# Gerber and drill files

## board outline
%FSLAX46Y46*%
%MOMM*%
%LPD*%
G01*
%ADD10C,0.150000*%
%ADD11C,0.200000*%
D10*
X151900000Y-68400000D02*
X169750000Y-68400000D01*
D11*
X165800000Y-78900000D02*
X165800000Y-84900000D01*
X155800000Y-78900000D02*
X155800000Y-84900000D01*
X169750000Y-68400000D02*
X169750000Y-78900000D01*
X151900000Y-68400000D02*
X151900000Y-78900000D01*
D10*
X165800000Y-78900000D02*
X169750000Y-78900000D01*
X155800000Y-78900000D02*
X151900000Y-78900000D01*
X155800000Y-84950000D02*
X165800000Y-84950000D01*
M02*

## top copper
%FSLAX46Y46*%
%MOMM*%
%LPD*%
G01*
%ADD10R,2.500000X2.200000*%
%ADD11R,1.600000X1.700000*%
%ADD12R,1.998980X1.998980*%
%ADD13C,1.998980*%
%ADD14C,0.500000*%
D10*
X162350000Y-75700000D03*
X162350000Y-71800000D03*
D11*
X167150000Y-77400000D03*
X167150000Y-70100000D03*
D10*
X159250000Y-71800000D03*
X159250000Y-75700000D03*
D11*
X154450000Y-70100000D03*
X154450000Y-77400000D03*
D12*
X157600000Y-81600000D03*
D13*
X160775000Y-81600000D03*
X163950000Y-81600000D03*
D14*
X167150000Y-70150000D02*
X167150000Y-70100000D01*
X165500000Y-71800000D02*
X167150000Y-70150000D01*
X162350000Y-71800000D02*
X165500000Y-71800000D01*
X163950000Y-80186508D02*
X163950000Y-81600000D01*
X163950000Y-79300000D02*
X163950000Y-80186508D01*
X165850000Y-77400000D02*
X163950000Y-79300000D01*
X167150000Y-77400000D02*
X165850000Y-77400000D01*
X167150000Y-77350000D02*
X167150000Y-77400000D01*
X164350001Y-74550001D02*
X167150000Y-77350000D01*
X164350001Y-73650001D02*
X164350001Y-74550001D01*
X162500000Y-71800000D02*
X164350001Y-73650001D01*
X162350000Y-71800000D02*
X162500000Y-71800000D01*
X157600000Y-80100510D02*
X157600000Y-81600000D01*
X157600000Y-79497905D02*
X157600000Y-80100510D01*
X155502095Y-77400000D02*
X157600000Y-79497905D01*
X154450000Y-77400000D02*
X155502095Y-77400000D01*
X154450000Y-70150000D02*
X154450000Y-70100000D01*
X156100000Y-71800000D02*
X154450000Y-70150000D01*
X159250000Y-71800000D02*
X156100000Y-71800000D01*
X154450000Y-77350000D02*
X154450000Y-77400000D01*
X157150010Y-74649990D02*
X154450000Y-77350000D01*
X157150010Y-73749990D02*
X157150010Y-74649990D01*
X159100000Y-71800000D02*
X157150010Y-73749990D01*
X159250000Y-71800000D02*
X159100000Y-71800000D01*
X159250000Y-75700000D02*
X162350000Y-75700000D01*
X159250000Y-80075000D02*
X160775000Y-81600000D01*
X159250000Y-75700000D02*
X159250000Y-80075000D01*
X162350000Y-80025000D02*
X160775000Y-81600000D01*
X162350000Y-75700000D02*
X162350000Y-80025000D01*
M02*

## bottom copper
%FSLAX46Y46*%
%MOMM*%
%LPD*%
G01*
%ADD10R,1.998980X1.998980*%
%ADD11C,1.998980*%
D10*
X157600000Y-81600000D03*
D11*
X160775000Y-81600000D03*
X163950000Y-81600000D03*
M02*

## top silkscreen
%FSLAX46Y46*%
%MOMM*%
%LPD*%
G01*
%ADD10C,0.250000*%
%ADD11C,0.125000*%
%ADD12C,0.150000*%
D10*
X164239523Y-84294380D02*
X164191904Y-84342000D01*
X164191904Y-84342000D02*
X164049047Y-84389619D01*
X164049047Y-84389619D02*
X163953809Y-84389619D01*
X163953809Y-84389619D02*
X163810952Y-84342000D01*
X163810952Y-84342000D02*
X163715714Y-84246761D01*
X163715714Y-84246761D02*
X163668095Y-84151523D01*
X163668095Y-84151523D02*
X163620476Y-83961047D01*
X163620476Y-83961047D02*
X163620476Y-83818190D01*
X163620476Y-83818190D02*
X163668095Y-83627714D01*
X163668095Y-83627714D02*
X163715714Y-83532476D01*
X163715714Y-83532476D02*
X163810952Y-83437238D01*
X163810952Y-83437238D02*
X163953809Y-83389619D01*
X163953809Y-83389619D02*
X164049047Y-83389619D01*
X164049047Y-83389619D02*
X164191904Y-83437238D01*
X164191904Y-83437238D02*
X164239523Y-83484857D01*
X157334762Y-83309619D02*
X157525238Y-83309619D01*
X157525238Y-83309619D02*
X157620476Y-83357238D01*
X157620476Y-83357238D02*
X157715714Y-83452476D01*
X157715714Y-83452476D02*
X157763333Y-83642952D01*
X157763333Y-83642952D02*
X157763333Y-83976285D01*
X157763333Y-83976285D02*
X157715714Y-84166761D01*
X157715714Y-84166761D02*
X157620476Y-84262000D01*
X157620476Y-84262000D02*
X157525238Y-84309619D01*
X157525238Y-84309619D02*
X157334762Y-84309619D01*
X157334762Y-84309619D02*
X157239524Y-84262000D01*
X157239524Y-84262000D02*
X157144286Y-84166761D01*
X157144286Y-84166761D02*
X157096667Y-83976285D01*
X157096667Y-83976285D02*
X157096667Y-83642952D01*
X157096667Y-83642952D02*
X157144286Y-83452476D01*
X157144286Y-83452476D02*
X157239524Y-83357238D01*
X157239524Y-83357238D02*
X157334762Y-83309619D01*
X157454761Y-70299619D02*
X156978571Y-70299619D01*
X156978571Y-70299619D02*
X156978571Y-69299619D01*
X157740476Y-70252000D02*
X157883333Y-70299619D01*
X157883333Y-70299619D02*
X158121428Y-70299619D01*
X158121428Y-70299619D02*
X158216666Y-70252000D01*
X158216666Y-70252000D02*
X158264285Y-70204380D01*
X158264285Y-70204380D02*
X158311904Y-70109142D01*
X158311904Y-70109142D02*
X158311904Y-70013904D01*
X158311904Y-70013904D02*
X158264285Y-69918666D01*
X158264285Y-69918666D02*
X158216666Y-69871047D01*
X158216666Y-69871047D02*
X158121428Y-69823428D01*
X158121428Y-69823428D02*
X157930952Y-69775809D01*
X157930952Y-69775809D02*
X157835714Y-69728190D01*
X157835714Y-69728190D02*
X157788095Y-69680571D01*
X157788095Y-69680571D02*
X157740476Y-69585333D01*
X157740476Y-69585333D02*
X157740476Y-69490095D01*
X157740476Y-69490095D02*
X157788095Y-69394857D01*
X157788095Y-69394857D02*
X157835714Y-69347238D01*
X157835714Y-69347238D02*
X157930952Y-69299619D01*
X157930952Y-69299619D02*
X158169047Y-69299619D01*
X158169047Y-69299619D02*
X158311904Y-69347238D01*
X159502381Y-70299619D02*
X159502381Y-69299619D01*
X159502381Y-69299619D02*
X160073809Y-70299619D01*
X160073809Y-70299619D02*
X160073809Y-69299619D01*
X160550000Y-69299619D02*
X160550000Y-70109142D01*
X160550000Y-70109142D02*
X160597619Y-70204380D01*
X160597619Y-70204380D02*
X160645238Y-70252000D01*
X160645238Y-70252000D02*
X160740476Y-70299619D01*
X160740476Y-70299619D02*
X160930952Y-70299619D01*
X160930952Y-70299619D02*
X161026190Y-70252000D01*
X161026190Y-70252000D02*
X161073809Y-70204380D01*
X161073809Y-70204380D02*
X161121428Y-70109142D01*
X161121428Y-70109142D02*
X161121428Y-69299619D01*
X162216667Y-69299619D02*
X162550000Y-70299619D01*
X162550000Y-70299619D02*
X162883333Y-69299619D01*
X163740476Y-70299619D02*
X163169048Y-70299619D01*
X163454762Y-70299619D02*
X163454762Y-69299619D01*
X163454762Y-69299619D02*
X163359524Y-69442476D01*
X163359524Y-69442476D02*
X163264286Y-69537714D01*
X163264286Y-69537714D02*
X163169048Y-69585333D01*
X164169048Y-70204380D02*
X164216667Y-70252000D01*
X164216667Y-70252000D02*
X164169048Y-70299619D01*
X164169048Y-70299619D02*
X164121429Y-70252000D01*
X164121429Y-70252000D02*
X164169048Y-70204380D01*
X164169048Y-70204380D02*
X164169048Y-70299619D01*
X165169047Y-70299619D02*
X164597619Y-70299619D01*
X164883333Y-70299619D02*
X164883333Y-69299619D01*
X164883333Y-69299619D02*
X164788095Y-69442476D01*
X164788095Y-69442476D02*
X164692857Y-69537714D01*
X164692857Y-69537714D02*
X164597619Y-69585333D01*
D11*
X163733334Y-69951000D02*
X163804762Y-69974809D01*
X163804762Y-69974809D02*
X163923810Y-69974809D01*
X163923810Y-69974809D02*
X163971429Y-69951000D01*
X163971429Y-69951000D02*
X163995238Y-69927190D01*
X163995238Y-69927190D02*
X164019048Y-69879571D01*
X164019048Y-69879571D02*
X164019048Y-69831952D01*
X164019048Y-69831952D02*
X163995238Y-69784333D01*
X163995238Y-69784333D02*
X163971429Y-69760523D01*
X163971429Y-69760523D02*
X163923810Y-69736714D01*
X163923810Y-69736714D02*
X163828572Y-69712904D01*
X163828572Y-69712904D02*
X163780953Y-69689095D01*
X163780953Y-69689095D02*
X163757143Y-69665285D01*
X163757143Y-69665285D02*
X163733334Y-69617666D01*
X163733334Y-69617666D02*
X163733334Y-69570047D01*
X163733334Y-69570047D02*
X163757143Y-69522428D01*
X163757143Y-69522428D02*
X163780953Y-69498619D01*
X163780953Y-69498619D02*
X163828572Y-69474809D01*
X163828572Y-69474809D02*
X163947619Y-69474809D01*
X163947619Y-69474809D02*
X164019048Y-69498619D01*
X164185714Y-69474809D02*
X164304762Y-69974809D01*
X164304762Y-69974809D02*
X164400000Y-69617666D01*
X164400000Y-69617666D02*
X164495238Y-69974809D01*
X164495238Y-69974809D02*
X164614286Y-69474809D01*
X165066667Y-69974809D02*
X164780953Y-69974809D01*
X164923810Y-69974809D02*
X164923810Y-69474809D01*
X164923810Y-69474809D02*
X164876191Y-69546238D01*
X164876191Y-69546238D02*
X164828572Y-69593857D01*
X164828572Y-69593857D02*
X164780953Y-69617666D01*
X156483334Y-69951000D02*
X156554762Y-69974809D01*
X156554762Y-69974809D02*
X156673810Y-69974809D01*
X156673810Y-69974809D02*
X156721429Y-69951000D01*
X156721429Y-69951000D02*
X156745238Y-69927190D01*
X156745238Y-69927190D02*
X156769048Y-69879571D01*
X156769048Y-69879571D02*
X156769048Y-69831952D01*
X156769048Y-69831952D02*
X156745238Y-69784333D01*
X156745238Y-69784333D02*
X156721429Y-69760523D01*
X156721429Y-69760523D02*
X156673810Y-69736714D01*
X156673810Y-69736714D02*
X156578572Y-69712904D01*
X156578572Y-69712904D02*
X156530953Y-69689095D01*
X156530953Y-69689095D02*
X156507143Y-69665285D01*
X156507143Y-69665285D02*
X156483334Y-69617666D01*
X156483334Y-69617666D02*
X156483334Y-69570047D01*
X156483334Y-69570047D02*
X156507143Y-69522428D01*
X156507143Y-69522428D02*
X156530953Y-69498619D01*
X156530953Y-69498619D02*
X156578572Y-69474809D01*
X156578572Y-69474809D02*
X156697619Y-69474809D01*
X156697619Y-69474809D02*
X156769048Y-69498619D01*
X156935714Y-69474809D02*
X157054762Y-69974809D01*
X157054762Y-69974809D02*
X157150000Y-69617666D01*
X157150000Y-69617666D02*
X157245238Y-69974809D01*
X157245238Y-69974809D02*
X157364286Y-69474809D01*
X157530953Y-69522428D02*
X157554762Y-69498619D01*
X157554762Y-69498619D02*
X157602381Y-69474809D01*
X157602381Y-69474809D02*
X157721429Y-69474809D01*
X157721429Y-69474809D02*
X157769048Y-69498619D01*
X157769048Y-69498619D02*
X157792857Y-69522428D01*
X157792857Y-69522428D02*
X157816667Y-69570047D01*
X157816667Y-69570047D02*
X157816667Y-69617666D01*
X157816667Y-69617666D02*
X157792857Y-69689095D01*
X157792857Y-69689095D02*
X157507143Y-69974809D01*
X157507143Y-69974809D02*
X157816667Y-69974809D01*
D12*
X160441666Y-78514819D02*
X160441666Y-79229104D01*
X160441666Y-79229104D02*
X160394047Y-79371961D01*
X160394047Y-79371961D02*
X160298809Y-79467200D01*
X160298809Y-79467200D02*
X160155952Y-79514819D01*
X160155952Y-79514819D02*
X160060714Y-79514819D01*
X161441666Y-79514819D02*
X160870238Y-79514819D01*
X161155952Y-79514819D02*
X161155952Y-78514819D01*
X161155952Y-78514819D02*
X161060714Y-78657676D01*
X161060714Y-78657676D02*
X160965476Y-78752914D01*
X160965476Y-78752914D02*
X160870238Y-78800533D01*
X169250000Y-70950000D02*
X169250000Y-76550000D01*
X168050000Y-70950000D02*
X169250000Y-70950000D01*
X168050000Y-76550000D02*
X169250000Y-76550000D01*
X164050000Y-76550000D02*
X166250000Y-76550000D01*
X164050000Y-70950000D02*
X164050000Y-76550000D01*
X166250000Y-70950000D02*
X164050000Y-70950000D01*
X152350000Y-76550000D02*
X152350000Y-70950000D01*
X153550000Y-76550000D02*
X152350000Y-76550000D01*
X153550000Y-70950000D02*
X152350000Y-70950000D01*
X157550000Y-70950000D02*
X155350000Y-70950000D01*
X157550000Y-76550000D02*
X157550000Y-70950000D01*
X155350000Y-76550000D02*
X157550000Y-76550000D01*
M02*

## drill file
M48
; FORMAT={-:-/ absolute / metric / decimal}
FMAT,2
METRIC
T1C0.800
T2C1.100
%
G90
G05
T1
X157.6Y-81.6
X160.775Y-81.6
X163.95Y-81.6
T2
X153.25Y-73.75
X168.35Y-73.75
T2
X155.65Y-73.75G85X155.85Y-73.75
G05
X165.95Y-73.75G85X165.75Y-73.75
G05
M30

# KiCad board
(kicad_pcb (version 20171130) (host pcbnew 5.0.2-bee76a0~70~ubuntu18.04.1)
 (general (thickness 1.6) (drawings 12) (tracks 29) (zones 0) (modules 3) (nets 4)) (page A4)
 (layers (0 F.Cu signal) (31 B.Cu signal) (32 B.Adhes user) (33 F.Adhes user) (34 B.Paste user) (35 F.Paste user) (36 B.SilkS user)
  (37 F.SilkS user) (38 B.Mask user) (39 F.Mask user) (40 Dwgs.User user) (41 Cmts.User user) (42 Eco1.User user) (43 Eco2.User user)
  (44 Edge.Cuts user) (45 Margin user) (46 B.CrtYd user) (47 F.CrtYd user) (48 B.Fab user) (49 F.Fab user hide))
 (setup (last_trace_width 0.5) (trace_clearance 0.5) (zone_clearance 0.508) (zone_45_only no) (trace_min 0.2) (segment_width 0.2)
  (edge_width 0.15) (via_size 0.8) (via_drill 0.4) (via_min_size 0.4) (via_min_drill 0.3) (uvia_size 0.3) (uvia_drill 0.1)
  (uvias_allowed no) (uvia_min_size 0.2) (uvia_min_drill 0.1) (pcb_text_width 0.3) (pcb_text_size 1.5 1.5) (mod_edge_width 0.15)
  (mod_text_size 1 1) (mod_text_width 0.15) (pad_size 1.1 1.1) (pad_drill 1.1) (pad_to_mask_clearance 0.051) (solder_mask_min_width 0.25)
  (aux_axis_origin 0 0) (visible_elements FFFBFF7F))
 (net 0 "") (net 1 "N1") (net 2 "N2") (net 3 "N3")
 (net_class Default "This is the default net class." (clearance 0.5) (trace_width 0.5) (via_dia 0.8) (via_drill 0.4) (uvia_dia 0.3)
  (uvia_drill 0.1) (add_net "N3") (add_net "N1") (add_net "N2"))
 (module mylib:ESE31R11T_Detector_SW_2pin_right (layer F.Cu) (at 167.15 73.75 270)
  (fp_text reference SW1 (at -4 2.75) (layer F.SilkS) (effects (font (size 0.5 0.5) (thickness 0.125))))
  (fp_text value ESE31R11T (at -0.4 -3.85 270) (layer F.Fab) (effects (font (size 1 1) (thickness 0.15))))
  (fp_line (start -2.8 -2.1) (end 2.8 -2.1) (layer F.SilkS) (width 0.15))
  (fp_line (start -2.8 -0.9) (end -2.8 -2.1) (layer F.SilkS) (width 0.15))
  (fp_line (start 2.8 -0.9) (end 2.8 -2.1) (layer F.SilkS) (width 0.15))
  (fp_line (start 2.8 3.1) (end 2.8 0.9) (layer F.SilkS) (width 0.15))
  (fp_line (start -2.8 3.1) (end 2.8 3.1) (layer F.SilkS) (width 0.15))
  (fp_line (start -2.8 0.9) (end -2.8 3.1) (layer F.SilkS) (width 0.15))
  (pad 1 smd rect (at 1.95 4.8 270) (size 2.2 2.5) (layers F.Cu F.Paste F.Mask) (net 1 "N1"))
  (pad 2 smd rect (at -1.95 4.8 270) (size 2.2 2.5) (layers F.Cu F.Paste F.Mask) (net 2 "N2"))
  (pad "" np_thru_hole oval (at 0 1.3 270) (size 1.1 1.3) (drill oval 1.1 1.3) (layers *.Cu *.Mask))
  (pad "" np_thru_hole circle (at 0 -1.2 270) (size 1.1 1.1) (drill 1.1) (layers *.Cu *.Mask))
  (pad 2 smd rect (at 3.65 0 270) (size 1.7 1.6) (layers F.Cu F.Paste F.Mask) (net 2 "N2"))
  (pad 2 smd rect (at -3.65 0 270) (size 1.7 1.6) (layers F.Cu F.Paste F.Mask) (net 2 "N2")))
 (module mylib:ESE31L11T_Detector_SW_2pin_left (layer F.Cu) (at 154.45 73.75 90)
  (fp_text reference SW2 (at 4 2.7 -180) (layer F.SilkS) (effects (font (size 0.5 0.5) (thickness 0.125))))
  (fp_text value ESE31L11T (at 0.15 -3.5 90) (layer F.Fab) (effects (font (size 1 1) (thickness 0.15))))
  (fp_line (start -2.8 -2.1) (end 2.8 -2.1) (layer F.SilkS) (width 0.15))
  (fp_line (start -2.8 -0.9) (end -2.8 -2.1) (layer F.SilkS) (width 0.15))
  (fp_line (start 2.8 -0.9) (end 2.8 -2.1) (layer F.SilkS) (width 0.15))
  (fp_line (start 2.8 3.1) (end 2.8 0.9) (layer F.SilkS) (width 0.15))
  (fp_line (start -2.8 3.1) (end 2.8 3.1) (layer F.SilkS) (width 0.15))
  (fp_line (start -2.8 0.9) (end -2.8 3.1) (layer F.SilkS) (width 0.15))
  (pad 2 smd rect (at 1.95 4.8 90) (size 2.2 2.5) (layers F.Cu F.Paste F.Mask) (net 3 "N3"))
  (pad 1 smd rect (at -1.95 4.8 90) (size 2.2 2.5) (layers F.Cu F.Paste F.Mask) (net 1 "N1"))
  (pad "" np_thru_hole oval (at 0 1.3 90) (size 1.1 1.3) (drill oval 1.1 1.3) (layers *.Cu *.Mask))
  (pad "" np_thru_hole circle (at 0 -1.2 90) (size 1.1 1.1) (drill 1.1) (layers *.Cu *.Mask))
  (pad 2 smd rect (at 3.65 0 90) (size 1.7 1.6) (layers F.Cu F.Paste F.Mask) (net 3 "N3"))
  (pad 2 smd rect (at -3.65 0 90) (size 1.7 1.6) (layers F.Cu F.Paste F.Mask) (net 3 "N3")))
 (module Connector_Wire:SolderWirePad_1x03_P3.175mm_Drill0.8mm (layer F.Cu) (at 157.6 81.6)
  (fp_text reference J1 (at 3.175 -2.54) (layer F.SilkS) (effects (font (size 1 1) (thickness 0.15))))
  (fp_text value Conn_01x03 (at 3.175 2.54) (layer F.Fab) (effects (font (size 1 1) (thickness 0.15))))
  (pad 1 thru_hole rect (at 0 0) (size 1.99898 1.99898) (drill 0.8001) (layers *.Cu *.Mask) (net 3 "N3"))
  (pad 2 thru_hole circle (at 3.175 0) (size 1.99898 1.99898) (drill 0.8001) (layers *.Cu *.Mask) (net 1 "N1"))
  (pad 3 thru_hole circle (at 6.35 0) (size 1.99898 1.99898) (drill 0.8001) (layers *.Cu *.Mask) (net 2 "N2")))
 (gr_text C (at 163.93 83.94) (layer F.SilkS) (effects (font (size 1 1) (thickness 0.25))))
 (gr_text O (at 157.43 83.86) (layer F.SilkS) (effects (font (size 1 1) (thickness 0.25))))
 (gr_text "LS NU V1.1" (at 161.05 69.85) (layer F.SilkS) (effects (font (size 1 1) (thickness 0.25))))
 (gr_line (start 151.9 68.4) (end 169.75 68.4) (layer Edge.Cuts) (width 0.15))
 (gr_line (start 165.8 78.9) (end 165.8 84.9) (layer Edge.Cuts) (width 0.2))
 (gr_line (start 155.8 78.9) (end 155.8 84.9) (layer Edge.Cuts) (width 0.2))
 (gr_line (start 169.75 68.4) (end 169.75 78.9) (layer Edge.Cuts) (width 0.2))
 (gr_line (start 151.9 68.4) (end 151.9 78.9) (layer Edge.Cuts) (width 0.2))
 (gr_line (start 165.8 78.9) (end 169.75 78.9) (layer Edge.Cuts) (width 0.15))
 (gr_line (start 155.8 78.9) (end 151.9 78.9) (layer Edge.Cuts) (width 0.15))
 (gr_line (start 155.8 84.95) (end 165.8 84.95) (layer Edge.Cuts) (width 0.15))
 (segment (start 167.15 70.15) (end 167.15 70.1) (width 0.5) (layer F.Cu) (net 2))
 (segment (start 165.5 71.8) (end 167.15 70.15) (width 0.5) (layer F.Cu) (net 2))
 (segment (start 162.35 71.8) (end 165.5 71.8) (width 0.5) (layer F.Cu) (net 2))
 (segment (start 163.95 80.186508) (end 163.95 81.6) (width 0.5) (layer F.Cu) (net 2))
 (segment (start 163.95 79.3) (end 163.95 80.186508) (width 0.5) (layer F.Cu) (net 2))
 (segment (start 165.85 77.4) (end 163.95 79.3) (width 0.5) (layer F.Cu) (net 2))
 (segment (start 167.15 77.4) (end 165.85 77.4) (width 0.5) (layer F.Cu) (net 2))
 (segment (start 167.15 77.35) (end 167.15 77.4) (width 0.5) (layer F.Cu) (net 2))
 (segment (start 164.350001 74.550001) (end 167.15 77.35) (width 0.5) (layer F.Cu) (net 2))
 (segment (start 164.350001 73.650001) (end 164.350001 74.550001) (width 0.5) (layer F.Cu) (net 2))
 (segment (start 162.5 71.8) (end 164.350001 73.650001) (width 0.5) (layer F.Cu) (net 2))
 (segment (start 162.35 71.8) (end 162.5 71.8) (width 0.5) (layer F.Cu) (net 2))
 (segment (start 157.6 80.10051) (end 157.6 81.6) (width 0.5) (layer F.Cu) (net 3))
 (segment (start 157.6 79.497905) (end 157.6 80.10051) (width 0.5) (layer F.Cu) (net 3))
 (segment (start 155.502095 77.4) (end 157.6 79.497905) (width 0.5) (layer F.Cu) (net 3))
 (segment (start 154.45 77.4) (end 155.502095 77.4) (width 0.5) (layer F.Cu) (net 3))
 (segment (start 154.45 70.15) (end 154.45 70.1) (width 0.5) (layer F.Cu) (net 3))
 (segment (start 156.1 71.8) (end 154.45 70.15) (width 0.5) (layer F.Cu) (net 3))
 (segment (start 159.25 71.8) (end 156.1 71.8) (width 0.5) (layer F.Cu) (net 3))
 (segment (start 154.45 77.35) (end 154.45 77.4) (width 0.5) (layer F.Cu) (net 3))
 (segment (start 157.15001 74.64999) (end 154.45 77.35) (width 0.5) (layer F.Cu) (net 3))
 (segment (start 157.15001 73.74999) (end 157.15001 74.64999) (width 0.5) (layer F.Cu) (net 3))
 (segment (start 159.1 71.8) (end 157.15001 73.74999) (width 0.5) (layer F.Cu) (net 3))
 (segment (start 159.25 71.8) (end 159.1 71.8) (width 0.5) (layer F.Cu) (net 3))
 (segment (start 159.25 75.7) (end 162.35 75.7) (width 0.5) (layer F.Cu) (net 1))
 (segment (start 159.25 80.075) (end 160.775 81.6) (width 0.5) (layer F.Cu) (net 1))
 (segment (start 159.25 75.7) (end 159.25 80.075) (width 0.5) (layer F.Cu) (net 1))
 (segment (start 162.35 80.025) (end 160.775 81.6) (width 0.5) (layer F.Cu) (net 1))
 (segment (start 162.35 75.7) (end 162.35 80.025) (width 0.5) (layer F.Cu) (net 1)))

